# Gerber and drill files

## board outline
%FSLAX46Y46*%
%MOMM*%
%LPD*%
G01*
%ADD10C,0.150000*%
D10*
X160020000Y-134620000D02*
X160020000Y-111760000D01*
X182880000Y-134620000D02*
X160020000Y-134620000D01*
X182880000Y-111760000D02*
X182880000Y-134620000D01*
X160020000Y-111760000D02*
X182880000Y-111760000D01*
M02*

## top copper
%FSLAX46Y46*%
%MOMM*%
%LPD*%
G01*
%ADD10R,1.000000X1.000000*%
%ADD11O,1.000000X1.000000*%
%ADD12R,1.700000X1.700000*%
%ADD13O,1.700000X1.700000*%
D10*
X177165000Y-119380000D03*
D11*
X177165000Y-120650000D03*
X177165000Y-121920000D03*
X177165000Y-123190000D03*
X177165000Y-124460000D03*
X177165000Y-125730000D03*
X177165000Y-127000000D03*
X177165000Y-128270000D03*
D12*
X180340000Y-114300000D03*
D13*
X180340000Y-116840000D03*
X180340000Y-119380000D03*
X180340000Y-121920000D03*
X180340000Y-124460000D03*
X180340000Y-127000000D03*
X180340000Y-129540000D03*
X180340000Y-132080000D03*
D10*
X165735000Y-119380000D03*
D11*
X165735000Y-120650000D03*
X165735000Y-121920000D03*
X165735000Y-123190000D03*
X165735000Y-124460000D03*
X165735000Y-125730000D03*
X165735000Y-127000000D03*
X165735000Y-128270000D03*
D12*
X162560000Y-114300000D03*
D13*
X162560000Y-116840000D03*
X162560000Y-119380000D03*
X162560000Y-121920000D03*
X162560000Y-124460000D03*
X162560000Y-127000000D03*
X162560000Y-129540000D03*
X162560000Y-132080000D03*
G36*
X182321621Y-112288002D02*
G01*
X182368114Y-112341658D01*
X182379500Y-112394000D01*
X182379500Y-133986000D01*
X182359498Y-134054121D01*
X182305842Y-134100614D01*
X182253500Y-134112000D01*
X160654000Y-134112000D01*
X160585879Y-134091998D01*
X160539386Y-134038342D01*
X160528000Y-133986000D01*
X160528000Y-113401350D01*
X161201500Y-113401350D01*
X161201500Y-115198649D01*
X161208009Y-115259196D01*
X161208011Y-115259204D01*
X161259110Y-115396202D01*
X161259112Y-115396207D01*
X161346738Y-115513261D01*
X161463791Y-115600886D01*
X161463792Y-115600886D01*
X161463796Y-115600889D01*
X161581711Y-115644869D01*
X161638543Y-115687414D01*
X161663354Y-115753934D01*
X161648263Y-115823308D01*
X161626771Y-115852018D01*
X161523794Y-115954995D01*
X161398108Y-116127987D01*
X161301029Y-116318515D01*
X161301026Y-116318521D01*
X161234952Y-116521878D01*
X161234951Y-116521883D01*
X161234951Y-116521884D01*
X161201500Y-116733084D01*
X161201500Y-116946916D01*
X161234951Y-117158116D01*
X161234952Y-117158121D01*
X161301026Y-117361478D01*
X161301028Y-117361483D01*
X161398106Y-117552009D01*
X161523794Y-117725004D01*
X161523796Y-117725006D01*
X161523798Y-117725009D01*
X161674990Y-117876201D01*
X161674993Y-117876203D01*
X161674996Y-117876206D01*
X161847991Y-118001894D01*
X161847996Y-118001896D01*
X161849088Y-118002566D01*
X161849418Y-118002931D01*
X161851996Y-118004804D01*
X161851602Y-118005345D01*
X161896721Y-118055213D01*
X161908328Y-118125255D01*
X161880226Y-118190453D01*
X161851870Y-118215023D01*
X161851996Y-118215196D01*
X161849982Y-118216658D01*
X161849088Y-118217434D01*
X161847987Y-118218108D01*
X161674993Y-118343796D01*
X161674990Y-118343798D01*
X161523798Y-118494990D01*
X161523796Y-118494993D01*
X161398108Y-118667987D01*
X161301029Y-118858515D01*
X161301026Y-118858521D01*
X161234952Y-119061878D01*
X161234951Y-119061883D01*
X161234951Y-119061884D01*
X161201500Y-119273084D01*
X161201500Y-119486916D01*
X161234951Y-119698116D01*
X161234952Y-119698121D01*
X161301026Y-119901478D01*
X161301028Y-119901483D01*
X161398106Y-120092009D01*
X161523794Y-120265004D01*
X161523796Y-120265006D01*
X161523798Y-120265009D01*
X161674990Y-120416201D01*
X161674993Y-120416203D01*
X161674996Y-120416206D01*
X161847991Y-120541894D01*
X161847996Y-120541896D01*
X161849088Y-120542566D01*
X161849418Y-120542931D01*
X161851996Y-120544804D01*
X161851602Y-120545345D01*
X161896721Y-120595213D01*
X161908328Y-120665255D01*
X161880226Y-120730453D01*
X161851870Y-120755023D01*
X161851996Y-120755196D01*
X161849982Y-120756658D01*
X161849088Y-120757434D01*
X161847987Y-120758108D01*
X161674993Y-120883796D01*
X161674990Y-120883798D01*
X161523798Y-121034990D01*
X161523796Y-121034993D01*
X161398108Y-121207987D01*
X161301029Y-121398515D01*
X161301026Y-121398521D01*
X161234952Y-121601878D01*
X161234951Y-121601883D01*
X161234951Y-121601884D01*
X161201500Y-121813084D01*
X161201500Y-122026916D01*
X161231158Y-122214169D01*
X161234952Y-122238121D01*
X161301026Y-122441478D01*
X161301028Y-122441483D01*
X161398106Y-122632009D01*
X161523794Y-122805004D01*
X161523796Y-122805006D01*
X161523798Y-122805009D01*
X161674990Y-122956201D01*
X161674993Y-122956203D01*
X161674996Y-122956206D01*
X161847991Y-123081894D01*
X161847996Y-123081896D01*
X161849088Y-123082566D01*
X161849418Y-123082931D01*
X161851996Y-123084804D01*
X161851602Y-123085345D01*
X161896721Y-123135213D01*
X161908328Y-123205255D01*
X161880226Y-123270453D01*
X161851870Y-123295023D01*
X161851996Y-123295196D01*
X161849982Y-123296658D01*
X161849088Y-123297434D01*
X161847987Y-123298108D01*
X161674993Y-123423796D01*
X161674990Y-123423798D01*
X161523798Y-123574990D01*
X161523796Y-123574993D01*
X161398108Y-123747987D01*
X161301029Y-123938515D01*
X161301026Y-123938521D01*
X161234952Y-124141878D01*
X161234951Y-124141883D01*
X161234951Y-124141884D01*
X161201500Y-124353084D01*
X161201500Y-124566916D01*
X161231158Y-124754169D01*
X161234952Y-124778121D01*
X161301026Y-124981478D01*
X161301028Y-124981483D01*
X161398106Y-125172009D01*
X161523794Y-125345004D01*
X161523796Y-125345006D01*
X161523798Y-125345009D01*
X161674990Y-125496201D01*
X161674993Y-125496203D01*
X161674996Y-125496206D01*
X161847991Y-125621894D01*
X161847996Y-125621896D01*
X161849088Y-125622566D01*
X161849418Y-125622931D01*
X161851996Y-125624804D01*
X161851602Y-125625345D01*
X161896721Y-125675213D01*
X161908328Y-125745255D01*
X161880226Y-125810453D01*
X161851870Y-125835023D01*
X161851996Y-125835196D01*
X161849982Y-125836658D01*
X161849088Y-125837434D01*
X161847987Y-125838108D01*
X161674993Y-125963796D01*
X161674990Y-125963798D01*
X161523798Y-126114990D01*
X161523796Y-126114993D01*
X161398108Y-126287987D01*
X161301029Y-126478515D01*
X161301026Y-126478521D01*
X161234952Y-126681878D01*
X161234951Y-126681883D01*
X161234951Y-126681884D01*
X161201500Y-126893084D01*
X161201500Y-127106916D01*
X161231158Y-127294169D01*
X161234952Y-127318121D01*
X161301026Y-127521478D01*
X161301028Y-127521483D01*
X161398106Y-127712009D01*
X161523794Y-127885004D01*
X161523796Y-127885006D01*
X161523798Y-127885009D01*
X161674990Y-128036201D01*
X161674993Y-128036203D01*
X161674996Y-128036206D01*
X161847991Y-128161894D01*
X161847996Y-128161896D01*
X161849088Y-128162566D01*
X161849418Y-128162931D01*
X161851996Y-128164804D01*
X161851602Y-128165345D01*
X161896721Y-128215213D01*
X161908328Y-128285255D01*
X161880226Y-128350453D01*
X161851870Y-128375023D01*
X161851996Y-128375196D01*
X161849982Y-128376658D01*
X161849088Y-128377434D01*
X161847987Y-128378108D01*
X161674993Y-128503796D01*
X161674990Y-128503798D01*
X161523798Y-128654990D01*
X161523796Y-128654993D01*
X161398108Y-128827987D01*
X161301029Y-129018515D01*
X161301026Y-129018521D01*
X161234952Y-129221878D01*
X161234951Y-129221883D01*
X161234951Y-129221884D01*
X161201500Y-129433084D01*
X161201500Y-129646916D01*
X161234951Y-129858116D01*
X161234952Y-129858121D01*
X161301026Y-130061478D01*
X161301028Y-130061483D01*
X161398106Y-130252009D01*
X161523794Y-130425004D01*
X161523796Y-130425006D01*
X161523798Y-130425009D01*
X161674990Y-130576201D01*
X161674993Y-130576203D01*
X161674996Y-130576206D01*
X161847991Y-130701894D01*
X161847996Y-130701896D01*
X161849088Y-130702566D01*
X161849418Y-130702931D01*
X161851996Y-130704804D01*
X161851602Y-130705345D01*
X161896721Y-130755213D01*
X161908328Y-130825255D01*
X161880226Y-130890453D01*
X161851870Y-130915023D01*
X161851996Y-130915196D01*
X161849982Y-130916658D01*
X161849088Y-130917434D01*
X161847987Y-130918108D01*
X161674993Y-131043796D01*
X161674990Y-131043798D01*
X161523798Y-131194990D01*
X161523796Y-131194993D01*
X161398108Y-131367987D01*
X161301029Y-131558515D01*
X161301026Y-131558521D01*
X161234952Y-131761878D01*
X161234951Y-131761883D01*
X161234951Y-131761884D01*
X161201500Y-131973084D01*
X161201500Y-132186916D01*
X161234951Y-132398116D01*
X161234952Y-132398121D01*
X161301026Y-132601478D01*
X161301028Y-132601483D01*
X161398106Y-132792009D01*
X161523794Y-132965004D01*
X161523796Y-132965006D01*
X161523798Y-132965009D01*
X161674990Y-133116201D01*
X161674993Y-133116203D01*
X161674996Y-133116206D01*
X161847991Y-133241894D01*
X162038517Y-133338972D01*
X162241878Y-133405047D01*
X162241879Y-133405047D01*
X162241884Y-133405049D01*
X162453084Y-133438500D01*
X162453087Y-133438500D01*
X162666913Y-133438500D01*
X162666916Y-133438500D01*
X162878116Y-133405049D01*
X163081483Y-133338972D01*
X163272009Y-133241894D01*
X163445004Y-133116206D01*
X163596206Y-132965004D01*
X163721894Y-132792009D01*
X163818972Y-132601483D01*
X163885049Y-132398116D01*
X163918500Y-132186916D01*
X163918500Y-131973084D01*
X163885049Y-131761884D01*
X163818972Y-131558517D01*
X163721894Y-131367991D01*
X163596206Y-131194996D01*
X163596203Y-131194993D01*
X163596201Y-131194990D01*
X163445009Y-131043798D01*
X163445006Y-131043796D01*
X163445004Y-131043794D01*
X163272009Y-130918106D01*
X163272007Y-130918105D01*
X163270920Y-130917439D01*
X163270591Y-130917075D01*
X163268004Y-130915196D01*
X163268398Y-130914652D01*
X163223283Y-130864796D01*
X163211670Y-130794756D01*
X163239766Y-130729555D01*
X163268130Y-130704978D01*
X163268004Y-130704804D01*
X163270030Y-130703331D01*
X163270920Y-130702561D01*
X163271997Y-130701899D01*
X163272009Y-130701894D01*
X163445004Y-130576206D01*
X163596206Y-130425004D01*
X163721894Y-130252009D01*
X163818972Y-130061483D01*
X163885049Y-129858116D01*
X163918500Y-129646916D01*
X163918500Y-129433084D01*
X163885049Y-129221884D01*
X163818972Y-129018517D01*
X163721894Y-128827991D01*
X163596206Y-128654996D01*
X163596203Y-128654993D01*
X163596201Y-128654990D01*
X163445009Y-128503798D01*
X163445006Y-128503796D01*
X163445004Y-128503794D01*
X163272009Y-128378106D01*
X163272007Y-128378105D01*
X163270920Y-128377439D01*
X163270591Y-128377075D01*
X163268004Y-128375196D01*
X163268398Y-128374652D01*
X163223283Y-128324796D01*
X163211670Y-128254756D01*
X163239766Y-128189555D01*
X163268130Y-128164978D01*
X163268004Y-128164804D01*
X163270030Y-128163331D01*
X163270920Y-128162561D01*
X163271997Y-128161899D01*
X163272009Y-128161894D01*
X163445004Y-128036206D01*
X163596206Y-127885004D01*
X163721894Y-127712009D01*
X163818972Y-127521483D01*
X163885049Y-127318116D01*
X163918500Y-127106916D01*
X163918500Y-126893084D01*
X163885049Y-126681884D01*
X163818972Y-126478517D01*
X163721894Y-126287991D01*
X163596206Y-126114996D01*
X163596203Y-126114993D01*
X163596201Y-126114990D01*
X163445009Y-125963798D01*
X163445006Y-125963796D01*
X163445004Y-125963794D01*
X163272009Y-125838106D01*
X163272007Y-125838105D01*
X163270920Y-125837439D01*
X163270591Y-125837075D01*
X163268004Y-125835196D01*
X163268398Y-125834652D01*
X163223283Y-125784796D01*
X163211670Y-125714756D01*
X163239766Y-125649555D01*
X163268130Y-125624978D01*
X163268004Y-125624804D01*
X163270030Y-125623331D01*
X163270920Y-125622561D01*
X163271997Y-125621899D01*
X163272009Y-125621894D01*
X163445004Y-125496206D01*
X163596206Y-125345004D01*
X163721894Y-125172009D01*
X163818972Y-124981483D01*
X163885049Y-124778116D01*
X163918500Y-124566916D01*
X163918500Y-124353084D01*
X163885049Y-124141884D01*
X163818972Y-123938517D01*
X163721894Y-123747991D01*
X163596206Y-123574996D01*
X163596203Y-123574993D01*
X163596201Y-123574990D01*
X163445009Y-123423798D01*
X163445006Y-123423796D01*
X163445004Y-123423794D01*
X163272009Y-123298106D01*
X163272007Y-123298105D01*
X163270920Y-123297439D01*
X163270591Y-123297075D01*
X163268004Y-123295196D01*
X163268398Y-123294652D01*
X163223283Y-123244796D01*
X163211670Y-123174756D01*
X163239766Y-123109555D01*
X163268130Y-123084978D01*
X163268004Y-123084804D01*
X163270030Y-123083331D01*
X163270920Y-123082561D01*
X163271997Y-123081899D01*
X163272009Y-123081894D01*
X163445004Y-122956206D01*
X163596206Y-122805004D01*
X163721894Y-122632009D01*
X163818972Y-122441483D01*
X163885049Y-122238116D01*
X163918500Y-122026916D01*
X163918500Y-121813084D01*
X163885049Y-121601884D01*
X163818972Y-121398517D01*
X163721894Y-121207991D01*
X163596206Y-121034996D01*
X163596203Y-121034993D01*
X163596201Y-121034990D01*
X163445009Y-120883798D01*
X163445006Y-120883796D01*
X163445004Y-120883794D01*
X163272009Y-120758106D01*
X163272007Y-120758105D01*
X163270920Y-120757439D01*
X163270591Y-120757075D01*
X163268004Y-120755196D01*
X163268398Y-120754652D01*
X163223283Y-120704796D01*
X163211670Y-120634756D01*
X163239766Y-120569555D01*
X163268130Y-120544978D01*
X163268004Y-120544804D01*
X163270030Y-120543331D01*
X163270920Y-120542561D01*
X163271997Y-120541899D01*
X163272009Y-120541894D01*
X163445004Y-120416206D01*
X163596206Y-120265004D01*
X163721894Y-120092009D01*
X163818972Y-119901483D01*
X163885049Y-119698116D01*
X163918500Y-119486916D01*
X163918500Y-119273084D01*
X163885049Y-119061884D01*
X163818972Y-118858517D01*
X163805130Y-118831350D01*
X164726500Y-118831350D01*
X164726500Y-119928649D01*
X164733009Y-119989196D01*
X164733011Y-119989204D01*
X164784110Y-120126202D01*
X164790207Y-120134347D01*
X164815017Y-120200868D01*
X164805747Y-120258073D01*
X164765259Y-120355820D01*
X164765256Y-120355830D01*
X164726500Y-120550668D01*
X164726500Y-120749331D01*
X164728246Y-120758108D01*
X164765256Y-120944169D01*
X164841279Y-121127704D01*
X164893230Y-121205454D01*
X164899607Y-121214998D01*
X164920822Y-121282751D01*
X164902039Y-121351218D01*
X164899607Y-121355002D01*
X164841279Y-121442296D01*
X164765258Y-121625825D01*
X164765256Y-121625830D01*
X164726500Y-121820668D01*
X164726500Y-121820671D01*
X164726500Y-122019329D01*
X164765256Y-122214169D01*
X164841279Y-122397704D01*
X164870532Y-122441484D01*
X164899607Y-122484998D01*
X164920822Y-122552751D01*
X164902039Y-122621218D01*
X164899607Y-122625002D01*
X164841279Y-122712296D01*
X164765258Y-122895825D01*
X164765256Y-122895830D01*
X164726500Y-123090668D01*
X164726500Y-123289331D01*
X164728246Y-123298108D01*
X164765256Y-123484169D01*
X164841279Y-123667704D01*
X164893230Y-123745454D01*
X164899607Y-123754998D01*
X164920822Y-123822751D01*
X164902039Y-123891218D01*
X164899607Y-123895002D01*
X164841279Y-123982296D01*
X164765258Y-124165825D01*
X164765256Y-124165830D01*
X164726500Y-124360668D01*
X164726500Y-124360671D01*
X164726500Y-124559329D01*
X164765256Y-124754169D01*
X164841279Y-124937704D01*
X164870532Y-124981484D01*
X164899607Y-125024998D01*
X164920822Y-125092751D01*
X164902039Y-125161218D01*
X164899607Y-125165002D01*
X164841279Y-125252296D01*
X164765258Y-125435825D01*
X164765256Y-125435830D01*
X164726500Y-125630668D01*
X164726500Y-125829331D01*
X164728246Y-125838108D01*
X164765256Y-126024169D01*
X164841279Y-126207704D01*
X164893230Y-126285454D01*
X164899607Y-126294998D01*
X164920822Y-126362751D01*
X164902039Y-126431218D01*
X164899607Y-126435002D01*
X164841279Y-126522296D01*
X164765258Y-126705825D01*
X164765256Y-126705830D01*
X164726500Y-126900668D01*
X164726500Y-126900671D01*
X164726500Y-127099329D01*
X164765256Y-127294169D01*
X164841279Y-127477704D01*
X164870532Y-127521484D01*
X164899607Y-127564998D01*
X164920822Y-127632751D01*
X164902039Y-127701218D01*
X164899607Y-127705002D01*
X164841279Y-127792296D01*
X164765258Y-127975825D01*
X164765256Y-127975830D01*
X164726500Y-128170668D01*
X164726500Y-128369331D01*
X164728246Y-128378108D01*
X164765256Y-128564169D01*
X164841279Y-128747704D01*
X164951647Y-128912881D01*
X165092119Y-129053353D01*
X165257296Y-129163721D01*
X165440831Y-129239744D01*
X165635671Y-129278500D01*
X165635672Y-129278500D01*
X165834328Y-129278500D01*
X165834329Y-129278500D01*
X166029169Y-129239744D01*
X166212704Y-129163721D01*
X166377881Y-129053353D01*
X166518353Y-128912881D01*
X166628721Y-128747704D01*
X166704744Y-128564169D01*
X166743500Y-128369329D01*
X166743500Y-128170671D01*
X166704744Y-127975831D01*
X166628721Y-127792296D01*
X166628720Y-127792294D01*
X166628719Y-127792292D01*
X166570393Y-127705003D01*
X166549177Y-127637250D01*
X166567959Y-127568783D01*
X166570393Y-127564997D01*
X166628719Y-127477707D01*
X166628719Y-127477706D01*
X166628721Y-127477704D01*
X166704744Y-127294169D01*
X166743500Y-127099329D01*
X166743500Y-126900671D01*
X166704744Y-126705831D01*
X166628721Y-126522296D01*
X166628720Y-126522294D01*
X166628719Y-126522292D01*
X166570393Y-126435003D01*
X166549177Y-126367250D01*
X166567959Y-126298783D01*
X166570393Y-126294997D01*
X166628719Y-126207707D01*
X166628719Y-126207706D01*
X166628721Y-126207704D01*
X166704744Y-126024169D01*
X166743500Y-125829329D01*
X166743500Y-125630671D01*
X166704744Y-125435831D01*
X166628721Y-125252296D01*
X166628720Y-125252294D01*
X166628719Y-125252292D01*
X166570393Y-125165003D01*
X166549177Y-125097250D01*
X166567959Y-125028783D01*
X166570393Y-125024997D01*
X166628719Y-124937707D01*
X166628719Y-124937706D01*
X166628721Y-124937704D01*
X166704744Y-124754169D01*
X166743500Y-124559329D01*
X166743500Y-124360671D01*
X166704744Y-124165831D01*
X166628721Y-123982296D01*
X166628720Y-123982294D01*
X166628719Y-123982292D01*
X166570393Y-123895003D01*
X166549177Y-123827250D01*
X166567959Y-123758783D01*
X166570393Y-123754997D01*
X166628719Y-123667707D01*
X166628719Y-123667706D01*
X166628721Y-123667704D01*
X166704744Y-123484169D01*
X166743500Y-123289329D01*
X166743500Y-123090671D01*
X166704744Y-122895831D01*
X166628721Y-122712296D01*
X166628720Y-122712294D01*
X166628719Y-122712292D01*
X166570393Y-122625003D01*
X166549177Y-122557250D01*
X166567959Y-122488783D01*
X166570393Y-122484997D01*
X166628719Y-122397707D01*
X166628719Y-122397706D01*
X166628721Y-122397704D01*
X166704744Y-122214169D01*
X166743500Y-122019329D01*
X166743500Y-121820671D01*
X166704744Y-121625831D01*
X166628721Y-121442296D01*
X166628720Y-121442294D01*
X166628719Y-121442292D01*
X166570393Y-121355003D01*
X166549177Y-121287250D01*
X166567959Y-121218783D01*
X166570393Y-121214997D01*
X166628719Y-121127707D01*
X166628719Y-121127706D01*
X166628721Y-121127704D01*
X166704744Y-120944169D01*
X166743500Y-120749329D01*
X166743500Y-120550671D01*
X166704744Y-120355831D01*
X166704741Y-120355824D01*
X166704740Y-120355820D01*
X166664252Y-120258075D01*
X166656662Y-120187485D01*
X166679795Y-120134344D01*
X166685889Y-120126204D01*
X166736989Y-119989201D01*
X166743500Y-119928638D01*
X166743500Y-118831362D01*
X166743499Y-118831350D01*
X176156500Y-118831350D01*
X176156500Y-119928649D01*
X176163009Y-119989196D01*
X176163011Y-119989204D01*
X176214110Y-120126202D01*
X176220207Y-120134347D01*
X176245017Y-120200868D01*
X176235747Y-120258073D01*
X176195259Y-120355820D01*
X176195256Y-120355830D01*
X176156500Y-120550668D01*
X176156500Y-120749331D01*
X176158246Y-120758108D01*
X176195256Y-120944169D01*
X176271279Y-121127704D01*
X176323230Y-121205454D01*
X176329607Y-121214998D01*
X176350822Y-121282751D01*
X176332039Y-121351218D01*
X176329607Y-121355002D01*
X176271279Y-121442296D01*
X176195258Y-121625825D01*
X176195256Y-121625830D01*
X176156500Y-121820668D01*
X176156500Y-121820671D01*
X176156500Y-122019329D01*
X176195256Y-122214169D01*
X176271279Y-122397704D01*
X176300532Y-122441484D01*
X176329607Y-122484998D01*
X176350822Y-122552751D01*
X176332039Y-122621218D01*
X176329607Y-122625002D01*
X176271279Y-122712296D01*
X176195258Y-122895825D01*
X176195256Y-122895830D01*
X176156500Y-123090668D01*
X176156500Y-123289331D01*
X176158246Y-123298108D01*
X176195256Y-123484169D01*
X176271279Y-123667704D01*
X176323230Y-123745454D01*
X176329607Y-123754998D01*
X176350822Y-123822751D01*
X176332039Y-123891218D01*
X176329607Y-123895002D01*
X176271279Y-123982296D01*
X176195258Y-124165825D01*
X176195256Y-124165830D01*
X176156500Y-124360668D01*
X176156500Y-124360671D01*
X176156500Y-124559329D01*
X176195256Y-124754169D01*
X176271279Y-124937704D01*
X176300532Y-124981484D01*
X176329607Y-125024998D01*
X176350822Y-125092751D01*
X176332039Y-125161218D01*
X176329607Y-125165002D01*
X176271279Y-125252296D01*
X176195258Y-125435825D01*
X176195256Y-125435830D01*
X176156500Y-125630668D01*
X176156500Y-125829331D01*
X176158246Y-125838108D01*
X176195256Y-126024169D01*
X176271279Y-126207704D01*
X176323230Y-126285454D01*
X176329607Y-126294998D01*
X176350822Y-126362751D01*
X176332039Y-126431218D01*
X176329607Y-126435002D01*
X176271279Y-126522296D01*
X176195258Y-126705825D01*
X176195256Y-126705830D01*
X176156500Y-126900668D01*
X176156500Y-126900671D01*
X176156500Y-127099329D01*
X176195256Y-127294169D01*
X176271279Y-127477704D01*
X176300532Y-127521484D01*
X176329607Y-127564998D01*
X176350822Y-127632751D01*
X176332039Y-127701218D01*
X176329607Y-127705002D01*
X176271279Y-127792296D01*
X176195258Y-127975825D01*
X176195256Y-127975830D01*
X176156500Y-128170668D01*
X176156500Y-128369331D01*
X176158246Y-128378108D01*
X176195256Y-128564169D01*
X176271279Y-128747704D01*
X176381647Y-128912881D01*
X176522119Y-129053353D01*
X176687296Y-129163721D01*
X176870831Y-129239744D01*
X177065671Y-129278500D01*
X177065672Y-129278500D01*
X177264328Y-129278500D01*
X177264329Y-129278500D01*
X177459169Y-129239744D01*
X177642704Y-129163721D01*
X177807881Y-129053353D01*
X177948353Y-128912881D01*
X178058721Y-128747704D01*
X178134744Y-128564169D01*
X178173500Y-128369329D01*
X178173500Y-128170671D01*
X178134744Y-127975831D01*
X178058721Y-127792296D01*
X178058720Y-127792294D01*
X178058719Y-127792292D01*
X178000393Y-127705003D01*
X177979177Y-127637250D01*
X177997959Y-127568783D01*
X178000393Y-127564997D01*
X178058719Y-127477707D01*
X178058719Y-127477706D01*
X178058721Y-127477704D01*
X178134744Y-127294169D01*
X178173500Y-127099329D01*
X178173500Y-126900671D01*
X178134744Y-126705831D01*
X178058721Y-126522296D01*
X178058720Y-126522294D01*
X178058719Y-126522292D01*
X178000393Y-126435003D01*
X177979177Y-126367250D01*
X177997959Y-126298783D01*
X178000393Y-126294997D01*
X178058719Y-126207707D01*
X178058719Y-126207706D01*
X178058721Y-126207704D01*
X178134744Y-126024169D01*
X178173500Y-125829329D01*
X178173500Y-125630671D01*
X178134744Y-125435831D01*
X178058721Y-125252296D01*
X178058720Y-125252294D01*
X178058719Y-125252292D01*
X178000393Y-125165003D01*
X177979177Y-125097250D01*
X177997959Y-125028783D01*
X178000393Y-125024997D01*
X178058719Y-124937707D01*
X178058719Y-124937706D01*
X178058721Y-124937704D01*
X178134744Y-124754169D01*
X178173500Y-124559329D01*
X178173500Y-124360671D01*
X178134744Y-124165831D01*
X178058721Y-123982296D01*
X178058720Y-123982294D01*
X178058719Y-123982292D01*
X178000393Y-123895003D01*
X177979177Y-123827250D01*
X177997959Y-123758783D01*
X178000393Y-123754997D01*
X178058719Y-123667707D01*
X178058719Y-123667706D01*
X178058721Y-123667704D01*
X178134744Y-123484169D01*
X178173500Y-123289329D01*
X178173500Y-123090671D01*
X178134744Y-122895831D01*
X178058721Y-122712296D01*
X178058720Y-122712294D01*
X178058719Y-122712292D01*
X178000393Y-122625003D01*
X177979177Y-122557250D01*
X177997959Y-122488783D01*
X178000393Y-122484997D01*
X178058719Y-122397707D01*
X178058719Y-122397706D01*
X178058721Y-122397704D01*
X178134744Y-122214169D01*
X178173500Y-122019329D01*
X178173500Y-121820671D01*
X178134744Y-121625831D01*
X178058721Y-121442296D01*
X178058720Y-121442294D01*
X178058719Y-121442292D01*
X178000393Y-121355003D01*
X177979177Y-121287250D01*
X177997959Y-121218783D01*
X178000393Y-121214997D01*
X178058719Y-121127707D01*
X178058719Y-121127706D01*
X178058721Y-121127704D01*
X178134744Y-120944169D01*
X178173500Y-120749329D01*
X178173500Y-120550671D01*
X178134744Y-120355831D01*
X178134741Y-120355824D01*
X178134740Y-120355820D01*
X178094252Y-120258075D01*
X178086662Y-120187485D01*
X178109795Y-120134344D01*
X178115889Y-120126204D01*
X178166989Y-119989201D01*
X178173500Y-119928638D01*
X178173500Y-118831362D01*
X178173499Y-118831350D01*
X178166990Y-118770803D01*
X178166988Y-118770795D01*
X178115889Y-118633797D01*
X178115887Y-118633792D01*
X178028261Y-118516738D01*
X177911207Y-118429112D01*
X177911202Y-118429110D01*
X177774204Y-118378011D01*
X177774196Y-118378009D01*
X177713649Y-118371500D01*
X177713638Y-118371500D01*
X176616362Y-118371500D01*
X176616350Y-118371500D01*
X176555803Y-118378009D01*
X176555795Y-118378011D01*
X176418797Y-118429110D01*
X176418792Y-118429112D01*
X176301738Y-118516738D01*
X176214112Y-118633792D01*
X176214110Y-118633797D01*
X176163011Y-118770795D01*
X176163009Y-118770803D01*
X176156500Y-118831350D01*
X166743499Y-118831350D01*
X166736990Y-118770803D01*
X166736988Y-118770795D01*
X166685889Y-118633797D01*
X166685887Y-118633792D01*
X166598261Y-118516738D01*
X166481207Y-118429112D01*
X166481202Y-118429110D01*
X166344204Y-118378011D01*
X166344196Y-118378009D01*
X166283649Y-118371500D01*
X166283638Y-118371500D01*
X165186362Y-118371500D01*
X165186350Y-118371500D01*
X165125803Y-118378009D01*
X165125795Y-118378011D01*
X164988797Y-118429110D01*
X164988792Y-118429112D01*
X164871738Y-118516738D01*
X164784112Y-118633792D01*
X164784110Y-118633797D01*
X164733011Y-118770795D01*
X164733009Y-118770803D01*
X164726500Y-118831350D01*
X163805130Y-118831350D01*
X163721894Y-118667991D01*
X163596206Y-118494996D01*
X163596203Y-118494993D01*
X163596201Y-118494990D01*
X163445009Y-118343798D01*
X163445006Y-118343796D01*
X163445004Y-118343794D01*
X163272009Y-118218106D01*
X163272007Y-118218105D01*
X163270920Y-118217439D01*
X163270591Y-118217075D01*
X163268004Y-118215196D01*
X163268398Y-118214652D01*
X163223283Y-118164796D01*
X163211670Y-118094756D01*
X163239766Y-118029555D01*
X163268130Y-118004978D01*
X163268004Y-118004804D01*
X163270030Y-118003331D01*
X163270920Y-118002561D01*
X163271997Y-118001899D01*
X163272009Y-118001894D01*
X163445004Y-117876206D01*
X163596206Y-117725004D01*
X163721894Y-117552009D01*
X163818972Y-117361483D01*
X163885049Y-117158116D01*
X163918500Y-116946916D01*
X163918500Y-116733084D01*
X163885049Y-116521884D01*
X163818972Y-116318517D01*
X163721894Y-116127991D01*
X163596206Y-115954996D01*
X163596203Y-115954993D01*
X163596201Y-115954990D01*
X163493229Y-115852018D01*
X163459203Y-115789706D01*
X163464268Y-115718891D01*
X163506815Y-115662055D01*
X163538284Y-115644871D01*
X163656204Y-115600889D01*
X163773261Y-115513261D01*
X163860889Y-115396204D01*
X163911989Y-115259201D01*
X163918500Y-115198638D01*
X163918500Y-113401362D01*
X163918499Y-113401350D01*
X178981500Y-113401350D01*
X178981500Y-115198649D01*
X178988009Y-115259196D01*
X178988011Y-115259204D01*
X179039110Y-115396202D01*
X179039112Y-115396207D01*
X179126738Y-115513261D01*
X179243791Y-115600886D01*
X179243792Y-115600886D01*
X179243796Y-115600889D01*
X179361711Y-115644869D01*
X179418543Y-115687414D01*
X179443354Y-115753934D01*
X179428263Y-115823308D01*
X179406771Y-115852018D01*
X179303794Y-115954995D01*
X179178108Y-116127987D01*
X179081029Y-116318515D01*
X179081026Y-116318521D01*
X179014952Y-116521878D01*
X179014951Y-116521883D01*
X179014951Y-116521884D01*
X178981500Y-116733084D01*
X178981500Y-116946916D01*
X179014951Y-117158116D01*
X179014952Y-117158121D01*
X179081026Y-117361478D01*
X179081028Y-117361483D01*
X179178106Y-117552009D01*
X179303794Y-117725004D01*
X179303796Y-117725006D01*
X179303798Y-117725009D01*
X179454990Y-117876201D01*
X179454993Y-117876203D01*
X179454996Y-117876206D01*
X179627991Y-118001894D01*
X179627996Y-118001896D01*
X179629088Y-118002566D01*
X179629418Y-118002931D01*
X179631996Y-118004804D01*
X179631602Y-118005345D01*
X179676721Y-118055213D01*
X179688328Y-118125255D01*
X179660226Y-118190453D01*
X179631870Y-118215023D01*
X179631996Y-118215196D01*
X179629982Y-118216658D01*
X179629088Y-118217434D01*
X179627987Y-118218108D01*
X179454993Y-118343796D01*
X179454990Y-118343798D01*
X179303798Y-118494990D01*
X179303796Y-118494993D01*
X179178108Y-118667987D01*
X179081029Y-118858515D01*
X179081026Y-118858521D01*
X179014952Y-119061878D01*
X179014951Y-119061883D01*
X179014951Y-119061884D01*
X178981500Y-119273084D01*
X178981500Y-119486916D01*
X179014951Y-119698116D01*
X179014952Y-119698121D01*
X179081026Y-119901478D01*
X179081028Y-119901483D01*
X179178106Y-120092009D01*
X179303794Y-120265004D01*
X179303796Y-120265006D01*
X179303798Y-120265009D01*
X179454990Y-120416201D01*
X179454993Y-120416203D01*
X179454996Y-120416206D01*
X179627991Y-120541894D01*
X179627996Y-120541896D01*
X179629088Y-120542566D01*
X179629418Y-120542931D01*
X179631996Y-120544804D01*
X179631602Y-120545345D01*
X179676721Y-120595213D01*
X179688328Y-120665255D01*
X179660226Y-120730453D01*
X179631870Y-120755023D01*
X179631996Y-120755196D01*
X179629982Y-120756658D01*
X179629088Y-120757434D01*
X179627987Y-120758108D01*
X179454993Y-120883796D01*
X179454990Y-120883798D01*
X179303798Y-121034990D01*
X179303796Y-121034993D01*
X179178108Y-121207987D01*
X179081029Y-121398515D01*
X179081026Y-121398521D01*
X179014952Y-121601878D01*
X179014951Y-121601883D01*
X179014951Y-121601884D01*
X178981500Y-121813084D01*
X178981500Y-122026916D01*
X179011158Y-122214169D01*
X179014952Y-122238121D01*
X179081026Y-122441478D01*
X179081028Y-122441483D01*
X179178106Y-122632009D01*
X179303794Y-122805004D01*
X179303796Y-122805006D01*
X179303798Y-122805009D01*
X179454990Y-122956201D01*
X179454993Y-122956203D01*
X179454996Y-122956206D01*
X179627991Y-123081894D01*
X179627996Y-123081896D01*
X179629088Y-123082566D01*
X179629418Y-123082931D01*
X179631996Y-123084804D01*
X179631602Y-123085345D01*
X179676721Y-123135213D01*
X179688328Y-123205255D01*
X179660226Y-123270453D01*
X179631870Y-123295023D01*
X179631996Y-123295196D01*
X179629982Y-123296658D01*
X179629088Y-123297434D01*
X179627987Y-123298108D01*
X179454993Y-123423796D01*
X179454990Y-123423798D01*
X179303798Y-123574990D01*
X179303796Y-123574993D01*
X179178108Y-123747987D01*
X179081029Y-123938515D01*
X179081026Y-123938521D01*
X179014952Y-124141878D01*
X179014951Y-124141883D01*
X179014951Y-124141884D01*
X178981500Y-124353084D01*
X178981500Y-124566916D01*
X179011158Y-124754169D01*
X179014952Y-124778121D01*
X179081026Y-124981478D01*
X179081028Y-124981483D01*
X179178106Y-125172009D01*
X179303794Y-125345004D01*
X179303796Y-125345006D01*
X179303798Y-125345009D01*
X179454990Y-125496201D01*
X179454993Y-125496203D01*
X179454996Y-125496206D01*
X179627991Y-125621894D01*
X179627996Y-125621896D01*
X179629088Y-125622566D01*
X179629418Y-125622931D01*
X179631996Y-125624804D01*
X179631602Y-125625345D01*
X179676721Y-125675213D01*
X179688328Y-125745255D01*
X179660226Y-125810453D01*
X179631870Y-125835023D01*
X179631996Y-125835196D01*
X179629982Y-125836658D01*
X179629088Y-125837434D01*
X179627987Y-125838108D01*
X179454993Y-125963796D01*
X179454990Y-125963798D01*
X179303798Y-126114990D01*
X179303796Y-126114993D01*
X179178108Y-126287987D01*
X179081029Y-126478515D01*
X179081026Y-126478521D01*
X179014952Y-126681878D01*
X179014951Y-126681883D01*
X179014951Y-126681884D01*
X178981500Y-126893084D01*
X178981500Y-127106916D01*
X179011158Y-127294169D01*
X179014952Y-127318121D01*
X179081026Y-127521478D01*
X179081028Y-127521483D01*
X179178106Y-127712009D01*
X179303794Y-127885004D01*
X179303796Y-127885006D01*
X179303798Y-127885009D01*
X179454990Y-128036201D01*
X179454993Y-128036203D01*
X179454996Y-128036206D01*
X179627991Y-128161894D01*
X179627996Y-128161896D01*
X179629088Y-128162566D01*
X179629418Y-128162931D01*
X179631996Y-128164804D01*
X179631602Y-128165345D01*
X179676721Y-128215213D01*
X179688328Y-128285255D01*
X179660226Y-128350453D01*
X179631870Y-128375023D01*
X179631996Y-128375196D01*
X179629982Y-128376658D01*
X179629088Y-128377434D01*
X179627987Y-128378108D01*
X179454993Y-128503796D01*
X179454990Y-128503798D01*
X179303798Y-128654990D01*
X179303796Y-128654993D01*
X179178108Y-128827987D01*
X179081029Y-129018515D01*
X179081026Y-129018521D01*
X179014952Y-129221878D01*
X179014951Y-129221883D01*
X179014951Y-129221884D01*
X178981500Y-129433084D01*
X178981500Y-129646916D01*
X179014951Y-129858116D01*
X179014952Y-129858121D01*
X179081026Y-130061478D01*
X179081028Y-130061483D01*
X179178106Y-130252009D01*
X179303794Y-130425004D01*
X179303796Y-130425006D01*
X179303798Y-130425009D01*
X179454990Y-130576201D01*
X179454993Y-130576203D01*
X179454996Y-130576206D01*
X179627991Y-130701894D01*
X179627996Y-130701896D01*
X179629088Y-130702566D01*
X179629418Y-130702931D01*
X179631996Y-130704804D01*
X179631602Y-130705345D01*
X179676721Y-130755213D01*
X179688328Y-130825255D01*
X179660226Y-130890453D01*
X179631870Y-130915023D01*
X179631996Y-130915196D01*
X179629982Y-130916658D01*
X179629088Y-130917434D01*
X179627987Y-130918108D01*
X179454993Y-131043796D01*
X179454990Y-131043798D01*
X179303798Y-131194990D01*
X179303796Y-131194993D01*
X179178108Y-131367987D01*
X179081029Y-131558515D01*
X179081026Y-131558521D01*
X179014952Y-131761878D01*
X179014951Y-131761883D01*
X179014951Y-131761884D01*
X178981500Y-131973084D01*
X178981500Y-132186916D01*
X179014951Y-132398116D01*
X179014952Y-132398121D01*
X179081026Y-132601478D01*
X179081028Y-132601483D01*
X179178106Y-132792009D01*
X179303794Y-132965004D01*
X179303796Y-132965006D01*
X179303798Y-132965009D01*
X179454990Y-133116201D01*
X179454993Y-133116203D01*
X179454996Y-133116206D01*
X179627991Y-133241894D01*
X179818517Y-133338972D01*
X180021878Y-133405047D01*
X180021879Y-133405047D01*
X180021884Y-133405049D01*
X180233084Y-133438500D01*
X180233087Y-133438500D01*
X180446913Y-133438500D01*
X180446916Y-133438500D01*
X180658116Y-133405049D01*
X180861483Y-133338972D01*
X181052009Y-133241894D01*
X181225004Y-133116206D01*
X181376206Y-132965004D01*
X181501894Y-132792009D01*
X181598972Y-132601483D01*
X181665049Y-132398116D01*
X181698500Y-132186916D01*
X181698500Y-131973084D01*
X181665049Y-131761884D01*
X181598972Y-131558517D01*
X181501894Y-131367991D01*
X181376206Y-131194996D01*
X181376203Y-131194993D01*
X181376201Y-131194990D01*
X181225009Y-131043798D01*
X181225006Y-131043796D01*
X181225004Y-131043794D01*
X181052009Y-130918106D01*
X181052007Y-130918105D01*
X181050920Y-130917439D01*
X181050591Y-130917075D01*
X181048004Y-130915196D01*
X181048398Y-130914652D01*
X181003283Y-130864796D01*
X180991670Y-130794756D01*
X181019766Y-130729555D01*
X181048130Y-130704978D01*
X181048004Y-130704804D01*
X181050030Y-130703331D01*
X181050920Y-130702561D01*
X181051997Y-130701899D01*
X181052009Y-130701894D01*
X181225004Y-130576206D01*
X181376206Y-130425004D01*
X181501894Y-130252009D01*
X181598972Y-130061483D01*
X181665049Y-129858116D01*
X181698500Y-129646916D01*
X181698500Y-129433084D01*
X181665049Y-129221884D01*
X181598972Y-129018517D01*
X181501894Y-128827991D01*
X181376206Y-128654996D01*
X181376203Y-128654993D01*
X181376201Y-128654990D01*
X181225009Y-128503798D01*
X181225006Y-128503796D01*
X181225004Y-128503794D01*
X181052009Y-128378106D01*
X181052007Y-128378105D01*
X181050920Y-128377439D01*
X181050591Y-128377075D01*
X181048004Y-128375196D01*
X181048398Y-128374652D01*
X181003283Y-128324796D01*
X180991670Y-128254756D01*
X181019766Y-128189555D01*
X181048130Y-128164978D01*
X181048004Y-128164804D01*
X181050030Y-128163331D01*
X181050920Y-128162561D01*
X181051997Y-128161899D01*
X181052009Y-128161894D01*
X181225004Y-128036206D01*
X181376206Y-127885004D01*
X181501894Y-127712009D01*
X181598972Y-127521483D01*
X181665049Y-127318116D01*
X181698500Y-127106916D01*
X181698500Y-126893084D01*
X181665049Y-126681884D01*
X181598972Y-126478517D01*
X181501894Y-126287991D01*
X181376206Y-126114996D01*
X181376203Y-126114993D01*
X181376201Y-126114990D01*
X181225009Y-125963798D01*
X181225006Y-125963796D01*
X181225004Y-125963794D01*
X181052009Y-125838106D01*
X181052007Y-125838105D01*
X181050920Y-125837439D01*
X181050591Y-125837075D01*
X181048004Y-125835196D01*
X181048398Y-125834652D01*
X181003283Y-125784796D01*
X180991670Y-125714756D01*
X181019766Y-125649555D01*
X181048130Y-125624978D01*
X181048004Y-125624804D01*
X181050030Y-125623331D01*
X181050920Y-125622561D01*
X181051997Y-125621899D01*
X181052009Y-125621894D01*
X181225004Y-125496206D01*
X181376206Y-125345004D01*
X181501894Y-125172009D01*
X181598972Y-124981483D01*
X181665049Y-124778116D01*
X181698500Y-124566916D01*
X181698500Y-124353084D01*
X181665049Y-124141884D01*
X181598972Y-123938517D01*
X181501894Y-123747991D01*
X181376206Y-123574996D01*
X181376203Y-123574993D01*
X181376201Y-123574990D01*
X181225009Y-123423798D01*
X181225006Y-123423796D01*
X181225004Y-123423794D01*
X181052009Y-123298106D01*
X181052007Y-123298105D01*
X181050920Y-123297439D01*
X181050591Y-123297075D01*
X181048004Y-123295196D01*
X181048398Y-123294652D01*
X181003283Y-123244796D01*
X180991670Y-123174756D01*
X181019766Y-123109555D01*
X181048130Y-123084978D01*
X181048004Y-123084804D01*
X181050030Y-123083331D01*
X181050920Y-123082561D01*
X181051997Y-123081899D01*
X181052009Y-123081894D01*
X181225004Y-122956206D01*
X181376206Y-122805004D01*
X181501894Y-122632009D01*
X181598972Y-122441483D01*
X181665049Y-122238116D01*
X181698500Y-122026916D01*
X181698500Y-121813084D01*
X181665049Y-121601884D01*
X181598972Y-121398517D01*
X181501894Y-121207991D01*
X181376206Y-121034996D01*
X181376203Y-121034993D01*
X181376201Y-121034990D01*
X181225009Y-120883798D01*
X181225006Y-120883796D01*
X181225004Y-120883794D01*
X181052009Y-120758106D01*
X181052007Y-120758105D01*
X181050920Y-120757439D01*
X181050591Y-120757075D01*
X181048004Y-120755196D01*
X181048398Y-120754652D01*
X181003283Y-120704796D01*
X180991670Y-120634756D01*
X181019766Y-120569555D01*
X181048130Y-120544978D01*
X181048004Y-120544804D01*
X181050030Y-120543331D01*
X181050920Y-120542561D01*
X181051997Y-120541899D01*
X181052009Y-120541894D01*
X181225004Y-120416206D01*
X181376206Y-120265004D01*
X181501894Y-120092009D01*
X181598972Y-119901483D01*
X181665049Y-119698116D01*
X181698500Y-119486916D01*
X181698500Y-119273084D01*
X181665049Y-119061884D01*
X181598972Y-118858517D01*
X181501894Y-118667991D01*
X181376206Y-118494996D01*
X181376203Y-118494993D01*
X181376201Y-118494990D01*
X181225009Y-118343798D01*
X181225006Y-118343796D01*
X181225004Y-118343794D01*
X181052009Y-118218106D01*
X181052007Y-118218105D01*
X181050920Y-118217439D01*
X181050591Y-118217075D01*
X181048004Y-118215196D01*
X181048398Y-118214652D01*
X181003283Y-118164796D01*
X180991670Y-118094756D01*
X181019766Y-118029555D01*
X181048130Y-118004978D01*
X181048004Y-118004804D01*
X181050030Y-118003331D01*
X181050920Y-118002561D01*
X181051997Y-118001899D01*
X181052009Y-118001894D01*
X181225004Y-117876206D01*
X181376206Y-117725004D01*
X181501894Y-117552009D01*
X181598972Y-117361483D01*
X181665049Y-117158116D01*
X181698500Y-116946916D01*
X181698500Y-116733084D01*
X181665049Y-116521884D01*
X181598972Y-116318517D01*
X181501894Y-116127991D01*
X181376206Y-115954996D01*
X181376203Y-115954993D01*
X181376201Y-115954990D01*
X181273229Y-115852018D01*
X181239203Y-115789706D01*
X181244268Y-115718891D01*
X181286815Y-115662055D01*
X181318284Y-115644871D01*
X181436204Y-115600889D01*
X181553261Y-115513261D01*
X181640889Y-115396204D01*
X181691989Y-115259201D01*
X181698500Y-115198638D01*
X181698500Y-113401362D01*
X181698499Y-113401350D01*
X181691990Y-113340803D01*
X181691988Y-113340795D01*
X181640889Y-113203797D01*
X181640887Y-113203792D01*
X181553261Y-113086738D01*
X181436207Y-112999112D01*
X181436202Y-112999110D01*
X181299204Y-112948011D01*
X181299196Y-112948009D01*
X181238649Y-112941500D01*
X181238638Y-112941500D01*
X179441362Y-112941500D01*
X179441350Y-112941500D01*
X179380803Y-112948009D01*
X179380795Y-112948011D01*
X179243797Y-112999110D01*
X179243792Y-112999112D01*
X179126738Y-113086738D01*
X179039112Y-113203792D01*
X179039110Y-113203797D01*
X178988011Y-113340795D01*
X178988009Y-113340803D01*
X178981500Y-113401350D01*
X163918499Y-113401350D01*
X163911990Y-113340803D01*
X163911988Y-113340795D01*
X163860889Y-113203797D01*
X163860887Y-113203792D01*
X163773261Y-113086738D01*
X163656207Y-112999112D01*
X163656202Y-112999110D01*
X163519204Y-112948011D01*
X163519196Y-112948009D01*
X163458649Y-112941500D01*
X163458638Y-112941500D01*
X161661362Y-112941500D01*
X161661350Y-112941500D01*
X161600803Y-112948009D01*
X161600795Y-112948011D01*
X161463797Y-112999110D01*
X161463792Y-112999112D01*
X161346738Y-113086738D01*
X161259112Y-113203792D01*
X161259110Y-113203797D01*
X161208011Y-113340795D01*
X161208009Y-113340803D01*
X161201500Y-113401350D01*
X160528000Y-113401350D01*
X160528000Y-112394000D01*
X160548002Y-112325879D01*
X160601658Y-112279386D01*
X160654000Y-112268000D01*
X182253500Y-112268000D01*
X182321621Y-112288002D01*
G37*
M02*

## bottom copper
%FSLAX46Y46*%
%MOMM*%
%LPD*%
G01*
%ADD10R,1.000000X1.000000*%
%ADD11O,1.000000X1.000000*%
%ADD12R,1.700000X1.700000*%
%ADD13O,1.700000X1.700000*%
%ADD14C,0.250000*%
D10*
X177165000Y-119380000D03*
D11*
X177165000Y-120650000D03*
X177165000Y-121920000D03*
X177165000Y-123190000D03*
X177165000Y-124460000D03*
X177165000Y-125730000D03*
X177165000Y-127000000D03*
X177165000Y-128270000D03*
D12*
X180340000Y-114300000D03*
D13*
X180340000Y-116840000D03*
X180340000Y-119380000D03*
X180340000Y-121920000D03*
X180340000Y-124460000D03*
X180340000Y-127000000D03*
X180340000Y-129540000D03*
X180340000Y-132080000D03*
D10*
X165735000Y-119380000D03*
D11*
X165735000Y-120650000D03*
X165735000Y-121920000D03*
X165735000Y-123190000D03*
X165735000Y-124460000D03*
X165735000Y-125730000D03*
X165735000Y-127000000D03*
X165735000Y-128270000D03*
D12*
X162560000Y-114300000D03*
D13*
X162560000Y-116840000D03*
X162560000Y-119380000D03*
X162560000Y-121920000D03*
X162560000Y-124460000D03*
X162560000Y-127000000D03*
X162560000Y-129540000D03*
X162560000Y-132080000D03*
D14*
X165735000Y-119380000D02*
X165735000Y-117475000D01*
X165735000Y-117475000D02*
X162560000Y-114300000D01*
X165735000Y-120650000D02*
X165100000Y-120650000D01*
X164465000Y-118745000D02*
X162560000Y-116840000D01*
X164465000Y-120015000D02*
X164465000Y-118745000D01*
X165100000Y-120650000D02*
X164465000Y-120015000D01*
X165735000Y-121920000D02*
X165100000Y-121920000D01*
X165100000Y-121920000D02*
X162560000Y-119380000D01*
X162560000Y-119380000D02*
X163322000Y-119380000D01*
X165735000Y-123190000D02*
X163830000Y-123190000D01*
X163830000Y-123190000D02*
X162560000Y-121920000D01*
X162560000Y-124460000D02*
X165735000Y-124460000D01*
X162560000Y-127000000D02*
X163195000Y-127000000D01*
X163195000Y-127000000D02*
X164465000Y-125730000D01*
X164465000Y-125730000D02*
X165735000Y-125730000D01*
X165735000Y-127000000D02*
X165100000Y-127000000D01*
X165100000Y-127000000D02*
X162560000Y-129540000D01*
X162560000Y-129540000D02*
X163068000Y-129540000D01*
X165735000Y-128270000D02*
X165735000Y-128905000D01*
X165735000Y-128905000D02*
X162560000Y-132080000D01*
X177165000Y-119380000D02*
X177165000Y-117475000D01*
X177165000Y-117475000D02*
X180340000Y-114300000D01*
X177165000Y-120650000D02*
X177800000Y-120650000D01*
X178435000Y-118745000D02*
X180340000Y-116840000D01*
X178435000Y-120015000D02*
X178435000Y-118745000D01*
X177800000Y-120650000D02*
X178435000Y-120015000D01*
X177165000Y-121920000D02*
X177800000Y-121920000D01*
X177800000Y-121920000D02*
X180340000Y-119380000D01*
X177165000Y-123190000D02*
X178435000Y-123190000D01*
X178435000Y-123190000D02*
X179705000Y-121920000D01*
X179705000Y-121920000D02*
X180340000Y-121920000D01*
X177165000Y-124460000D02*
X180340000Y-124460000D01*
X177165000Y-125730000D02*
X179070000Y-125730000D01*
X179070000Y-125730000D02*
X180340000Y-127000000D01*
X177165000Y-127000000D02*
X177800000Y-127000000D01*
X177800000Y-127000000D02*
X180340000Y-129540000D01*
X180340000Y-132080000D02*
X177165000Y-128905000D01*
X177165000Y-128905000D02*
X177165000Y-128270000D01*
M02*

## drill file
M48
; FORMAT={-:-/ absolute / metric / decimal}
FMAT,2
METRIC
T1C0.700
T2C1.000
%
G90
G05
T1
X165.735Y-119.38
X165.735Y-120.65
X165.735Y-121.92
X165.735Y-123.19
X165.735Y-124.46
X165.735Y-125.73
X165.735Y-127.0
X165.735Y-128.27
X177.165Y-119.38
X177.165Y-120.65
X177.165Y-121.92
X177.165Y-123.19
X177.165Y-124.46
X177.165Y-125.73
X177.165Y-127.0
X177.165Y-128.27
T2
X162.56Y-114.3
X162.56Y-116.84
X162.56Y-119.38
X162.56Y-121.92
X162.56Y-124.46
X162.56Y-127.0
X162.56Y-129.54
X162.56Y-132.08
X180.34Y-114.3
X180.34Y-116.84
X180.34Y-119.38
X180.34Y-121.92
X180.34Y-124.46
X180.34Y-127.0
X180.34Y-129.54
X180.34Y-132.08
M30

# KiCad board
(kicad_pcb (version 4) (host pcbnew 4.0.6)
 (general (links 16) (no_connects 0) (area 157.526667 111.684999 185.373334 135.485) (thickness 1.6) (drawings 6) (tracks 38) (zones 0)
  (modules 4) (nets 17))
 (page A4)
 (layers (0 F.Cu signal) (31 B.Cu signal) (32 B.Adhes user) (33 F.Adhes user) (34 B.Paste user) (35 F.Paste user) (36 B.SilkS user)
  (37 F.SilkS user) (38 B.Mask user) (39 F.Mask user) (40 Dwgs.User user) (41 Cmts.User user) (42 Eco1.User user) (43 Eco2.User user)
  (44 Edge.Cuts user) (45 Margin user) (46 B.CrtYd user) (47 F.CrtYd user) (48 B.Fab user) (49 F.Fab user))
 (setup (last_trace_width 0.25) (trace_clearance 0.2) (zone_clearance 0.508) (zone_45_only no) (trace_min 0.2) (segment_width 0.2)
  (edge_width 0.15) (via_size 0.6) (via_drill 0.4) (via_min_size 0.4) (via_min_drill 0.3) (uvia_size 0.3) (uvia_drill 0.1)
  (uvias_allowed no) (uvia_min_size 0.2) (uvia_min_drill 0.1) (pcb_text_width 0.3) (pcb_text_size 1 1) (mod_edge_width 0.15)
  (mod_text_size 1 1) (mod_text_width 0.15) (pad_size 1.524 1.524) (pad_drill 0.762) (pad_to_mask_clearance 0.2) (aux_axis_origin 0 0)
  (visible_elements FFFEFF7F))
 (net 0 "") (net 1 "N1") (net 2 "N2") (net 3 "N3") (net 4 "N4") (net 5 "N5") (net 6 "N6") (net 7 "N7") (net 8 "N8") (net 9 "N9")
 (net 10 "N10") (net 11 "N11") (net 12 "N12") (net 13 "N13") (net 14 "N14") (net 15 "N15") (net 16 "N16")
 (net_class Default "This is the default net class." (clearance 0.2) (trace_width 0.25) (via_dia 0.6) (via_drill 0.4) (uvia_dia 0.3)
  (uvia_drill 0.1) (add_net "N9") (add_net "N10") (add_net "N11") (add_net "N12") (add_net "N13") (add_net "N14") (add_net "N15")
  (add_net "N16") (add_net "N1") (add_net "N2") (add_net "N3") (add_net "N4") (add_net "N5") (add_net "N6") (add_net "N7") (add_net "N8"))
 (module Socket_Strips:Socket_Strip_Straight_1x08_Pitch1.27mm (layer F.Cu) (at 177.165 119.38)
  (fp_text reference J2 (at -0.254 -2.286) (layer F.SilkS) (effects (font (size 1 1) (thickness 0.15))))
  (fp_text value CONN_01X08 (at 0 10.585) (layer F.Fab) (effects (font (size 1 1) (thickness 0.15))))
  (pad 1 thru_hole rect (at 0 0) (size 1 1) (drill 0.7) (layers *.Cu *.Mask) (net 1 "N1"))
  (pad 2 thru_hole oval (at 0 1.27) (size 1 1) (drill 0.7) (layers *.Cu *.Mask) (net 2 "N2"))
  (pad 3 thru_hole oval (at 0 2.54) (size 1 1) (drill 0.7) (layers *.Cu *.Mask) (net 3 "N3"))
  (pad 4 thru_hole oval (at 0 3.81) (size 1 1) (drill 0.7) (layers *.Cu *.Mask) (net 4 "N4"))
  (pad 5 thru_hole oval (at 0 5.08) (size 1 1) (drill 0.7) (layers *.Cu *.Mask) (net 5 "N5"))
  (pad 6 thru_hole oval (at 0 6.35) (size 1 1) (drill 0.7) (layers *.Cu *.Mask) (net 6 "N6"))
  (pad 7 thru_hole oval (at 0 7.62) (size 1 1) (drill 0.7) (layers *.Cu *.Mask) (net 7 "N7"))
  (pad 8 thru_hole oval (at 0 8.89) (size 1 1) (drill 0.7) (layers *.Cu *.Mask) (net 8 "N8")))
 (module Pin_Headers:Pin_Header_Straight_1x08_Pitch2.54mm (layer F.Cu) (at 180.34 114.3)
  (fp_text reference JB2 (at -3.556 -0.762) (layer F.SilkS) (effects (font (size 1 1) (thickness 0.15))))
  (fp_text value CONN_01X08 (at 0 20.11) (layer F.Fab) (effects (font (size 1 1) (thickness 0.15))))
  (pad 1 thru_hole rect (at 0 0) (size 1.7 1.7) (drill 1) (layers *.Cu *.Mask) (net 1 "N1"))
  (pad 2 thru_hole oval (at 0 2.54) (size 1.7 1.7) (drill 1) (layers *.Cu *.Mask) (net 2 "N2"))
  (pad 3 thru_hole oval (at 0 5.08) (size 1.7 1.7) (drill 1) (layers *.Cu *.Mask) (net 3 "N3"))
  (pad 4 thru_hole oval (at 0 7.62) (size 1.7 1.7) (drill 1) (layers *.Cu *.Mask) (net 4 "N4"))
  (pad 5 thru_hole oval (at 0 10.16) (size 1.7 1.7) (drill 1) (layers *.Cu *.Mask) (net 5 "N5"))
  (pad 6 thru_hole oval (at 0 12.7) (size 1.7 1.7) (drill 1) (layers *.Cu *.Mask) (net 6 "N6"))
  (pad 7 thru_hole oval (at 0 15.24) (size 1.7 1.7) (drill 1) (layers *.Cu *.Mask) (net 7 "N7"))
  (pad 8 thru_hole oval (at 0 17.78) (size 1.7 1.7) (drill 1) (layers *.Cu *.Mask) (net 8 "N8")))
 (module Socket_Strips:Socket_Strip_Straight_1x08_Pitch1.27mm (layer F.Cu) (at 165.735 119.38)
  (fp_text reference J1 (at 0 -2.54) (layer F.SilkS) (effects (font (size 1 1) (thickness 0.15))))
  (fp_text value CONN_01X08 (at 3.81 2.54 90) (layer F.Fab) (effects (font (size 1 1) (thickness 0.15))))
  (pad 1 thru_hole rect (at 0 0) (size 1 1) (drill 0.7) (layers *.Cu *.Mask) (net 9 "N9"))
  (pad 2 thru_hole oval (at 0 1.27) (size 1 1) (drill 0.7) (layers *.Cu *.Mask) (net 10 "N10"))
  (pad 3 thru_hole oval (at 0 2.54) (size 1 1) (drill 0.7) (layers *.Cu *.Mask) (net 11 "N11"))
  (pad 4 thru_hole oval (at 0 3.81) (size 1 1) (drill 0.7) (layers *.Cu *.Mask) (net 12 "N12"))
  (pad 5 thru_hole oval (at 0 5.08) (size 1 1) (drill 0.7) (layers *.Cu *.Mask) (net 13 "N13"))
  (pad 6 thru_hole oval (at 0 6.35) (size 1 1) (drill 0.7) (layers *.Cu *.Mask) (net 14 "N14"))
  (pad 7 thru_hole oval (at 0 7.62) (size 1 1) (drill 0.7) (layers *.Cu *.Mask) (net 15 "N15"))
  (pad 8 thru_hole oval (at 0 8.89) (size 1 1) (drill 0.7) (layers *.Cu *.Mask) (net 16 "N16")))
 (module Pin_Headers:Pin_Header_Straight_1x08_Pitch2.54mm (layer F.Cu) (at 162.56 114.3)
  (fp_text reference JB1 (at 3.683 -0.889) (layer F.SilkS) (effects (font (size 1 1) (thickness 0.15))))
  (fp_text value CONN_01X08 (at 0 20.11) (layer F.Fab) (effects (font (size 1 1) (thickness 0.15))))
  (pad 1 thru_hole rect (at 0 0) (size 1.7 1.7) (drill 1) (layers *.Cu *.Mask) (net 9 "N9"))
  (pad 2 thru_hole oval (at 0 2.54) (size 1.7 1.7) (drill 1) (layers *.Cu *.Mask) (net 10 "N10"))
  (pad 3 thru_hole oval (at 0 5.08) (size 1.7 1.7) (drill 1) (layers *.Cu *.Mask) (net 11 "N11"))
  (pad 4 thru_hole oval (at 0 7.62) (size 1.7 1.7) (drill 1) (layers *.Cu *.Mask) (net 12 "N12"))
  (pad 5 thru_hole oval (at 0 10.16) (size 1.7 1.7) (drill 1) (layers *.Cu *.Mask) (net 13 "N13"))
  (pad 6 thru_hole oval (at 0 12.7) (size 1.7 1.7) (drill 1) (layers *.Cu *.Mask) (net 14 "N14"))
  (pad 7 thru_hole oval (at 0 15.24) (size 1.7 1.7) (drill 1) (layers *.Cu *.Mask) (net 15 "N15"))
  (pad 8 thru_hole oval (at 0 17.78) (size 1.7 1.7) (drill 1) (layers *.Cu *.Mask) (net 16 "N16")))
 (gr_line (start 160.02 134.62) (end 160.02 111.76) (angle 90) (layer Edge.Cuts) (width 0.15))
 (gr_line (start 182.88 134.62) (end 160.02 134.62) (angle 90) (layer Edge.Cuts) (width 0.15))
 (gr_line (start 182.88 111.76) (end 182.88 134.62) (angle 90) (layer Edge.Cuts) (width 0.15))
 (gr_line (start 160.02 111.76) (end 182.88 111.76) (angle 90) (layer Edge.Cuts) (width 0.15))
 (segment (start 165.735 119.38) (end 165.735 117.475) (width 0.25) (layer B.Cu) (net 9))
 (segment (start 165.735 117.475) (end 162.56 114.3) (width 0.25) (layer B.Cu) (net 9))
 (segment (start 165.735 120.65) (end 165.1 120.65) (width 0.25) (layer B.Cu) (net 10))
 (segment (start 164.465 118.745) (end 162.56 116.84) (width 0.25) (layer B.Cu) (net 10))
 (segment (start 164.465 120.015) (end 164.465 118.745) (width 0.25) (layer B.Cu) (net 10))
 (segment (start 165.1 120.65) (end 164.465 120.015) (width 0.25) (layer B.Cu) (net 10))
 (segment (start 165.735 121.92) (end 165.1 121.92) (width 0.25) (layer B.Cu) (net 11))
 (segment (start 165.1 121.92) (end 162.56 119.38) (width 0.25) (layer B.Cu) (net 11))
 (segment (start 162.56 119.38) (end 163.322 119.38) (width 0.25) (layer B.Cu) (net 11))
 (segment (start 165.735 123.19) (end 163.83 123.19) (width 0.25) (layer B.Cu) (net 12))
 (segment (start 163.83 123.19) (end 162.56 121.92) (width 0.25) (layer B.Cu) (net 12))
 (segment (start 162.56 124.46) (end 165.735 124.46) (width 0.25) (layer B.Cu) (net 13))
 (segment (start 162.56 127) (end 163.195 127) (width 0.25) (layer B.Cu) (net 14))
 (segment (start 163.195 127) (end 164.465 125.73) (width 0.25) (layer B.Cu) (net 14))
 (segment (start 164.465 125.73) (end 165.735 125.73) (width 0.25) (layer B.Cu) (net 14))
 (segment (start 165.735 127) (end 165.1 127) (width 0.25) (layer B.Cu) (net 15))
 (segment (start 165.1 127) (end 162.56 129.54) (width 0.25) (layer B.Cu) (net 15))
 (segment (start 162.56 129.54) (end 163.068 129.54) (width 0.25) (layer B.Cu) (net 15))
 (segment (start 165.735 128.27) (end 165.735 128.905) (width 0.25) (layer B.Cu) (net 16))
 (segment (start 165.735 128.905) (end 162.56 132.08) (width 0.25) (layer B.Cu) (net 16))
 (segment (start 177.165 119.38) (end 177.165 117.475) (width 0.25) (layer B.Cu) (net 1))
 (segment (start 177.165 117.475) (end 180.34 114.3) (width 0.25) (layer B.Cu) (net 1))
 (segment (start 177.165 120.65) (end 177.8 120.65) (width 0.25) (layer B.Cu) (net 2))
 (segment (start 178.435 118.745) (end 180.34 116.84) (width 0.25) (layer B.Cu) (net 2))
 (segment (start 178.435 120.015) (end 178.435 118.745) (width 0.25) (layer B.Cu) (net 2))
 (segment (start 177.8 120.65) (end 178.435 120.015) (width 0.25) (layer B.Cu) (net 2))
 (segment (start 177.165 121.92) (end 177.8 121.92) (width 0.25) (layer B.Cu) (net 3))
 (segment (start 177.8 121.92) (end 180.34 119.38) (width 0.25) (layer B.Cu) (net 3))
 (segment (start 177.165 123.19) (end 178.435 123.19) (width 0.25) (layer B.Cu) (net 4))
 (segment (start 178.435 123.19) (end 179.705 121.92) (width 0.25) (layer B.Cu) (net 4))
 (segment (start 179.705 121.92) (end 180.34 121.92) (width 0.25) (layer B.Cu) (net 4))
 (segment (start 177.165 124.46) (end 180.34 124.46) (width 0.25) (layer B.Cu) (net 5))
 (segment (start 177.165 125.73) (end 179.07 125.73) (width 0.25) (layer B.Cu) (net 6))
 (segment (start 179.07 125.73) (end 180.34 127) (width 0.25) (layer B.Cu) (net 6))
 (segment (start 177.165 127) (end 177.8 127) (width 0.25) (layer B.Cu) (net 7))
 (segment (start 177.8 127) (end 180.34 129.54) (width 0.25) (layer B.Cu) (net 7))
 (segment (start 180.34 132.08) (end 177.165 128.905) (width 0.25) (layer B.Cu) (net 8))
 (segment (start 177.165 128.905) (end 177.165 128.27) (width 0.25) (layer B.Cu) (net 8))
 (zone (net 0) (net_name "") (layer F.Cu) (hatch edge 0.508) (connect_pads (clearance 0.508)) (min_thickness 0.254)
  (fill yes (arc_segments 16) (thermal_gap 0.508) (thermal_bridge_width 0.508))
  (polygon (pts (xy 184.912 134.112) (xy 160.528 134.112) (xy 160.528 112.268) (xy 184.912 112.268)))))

